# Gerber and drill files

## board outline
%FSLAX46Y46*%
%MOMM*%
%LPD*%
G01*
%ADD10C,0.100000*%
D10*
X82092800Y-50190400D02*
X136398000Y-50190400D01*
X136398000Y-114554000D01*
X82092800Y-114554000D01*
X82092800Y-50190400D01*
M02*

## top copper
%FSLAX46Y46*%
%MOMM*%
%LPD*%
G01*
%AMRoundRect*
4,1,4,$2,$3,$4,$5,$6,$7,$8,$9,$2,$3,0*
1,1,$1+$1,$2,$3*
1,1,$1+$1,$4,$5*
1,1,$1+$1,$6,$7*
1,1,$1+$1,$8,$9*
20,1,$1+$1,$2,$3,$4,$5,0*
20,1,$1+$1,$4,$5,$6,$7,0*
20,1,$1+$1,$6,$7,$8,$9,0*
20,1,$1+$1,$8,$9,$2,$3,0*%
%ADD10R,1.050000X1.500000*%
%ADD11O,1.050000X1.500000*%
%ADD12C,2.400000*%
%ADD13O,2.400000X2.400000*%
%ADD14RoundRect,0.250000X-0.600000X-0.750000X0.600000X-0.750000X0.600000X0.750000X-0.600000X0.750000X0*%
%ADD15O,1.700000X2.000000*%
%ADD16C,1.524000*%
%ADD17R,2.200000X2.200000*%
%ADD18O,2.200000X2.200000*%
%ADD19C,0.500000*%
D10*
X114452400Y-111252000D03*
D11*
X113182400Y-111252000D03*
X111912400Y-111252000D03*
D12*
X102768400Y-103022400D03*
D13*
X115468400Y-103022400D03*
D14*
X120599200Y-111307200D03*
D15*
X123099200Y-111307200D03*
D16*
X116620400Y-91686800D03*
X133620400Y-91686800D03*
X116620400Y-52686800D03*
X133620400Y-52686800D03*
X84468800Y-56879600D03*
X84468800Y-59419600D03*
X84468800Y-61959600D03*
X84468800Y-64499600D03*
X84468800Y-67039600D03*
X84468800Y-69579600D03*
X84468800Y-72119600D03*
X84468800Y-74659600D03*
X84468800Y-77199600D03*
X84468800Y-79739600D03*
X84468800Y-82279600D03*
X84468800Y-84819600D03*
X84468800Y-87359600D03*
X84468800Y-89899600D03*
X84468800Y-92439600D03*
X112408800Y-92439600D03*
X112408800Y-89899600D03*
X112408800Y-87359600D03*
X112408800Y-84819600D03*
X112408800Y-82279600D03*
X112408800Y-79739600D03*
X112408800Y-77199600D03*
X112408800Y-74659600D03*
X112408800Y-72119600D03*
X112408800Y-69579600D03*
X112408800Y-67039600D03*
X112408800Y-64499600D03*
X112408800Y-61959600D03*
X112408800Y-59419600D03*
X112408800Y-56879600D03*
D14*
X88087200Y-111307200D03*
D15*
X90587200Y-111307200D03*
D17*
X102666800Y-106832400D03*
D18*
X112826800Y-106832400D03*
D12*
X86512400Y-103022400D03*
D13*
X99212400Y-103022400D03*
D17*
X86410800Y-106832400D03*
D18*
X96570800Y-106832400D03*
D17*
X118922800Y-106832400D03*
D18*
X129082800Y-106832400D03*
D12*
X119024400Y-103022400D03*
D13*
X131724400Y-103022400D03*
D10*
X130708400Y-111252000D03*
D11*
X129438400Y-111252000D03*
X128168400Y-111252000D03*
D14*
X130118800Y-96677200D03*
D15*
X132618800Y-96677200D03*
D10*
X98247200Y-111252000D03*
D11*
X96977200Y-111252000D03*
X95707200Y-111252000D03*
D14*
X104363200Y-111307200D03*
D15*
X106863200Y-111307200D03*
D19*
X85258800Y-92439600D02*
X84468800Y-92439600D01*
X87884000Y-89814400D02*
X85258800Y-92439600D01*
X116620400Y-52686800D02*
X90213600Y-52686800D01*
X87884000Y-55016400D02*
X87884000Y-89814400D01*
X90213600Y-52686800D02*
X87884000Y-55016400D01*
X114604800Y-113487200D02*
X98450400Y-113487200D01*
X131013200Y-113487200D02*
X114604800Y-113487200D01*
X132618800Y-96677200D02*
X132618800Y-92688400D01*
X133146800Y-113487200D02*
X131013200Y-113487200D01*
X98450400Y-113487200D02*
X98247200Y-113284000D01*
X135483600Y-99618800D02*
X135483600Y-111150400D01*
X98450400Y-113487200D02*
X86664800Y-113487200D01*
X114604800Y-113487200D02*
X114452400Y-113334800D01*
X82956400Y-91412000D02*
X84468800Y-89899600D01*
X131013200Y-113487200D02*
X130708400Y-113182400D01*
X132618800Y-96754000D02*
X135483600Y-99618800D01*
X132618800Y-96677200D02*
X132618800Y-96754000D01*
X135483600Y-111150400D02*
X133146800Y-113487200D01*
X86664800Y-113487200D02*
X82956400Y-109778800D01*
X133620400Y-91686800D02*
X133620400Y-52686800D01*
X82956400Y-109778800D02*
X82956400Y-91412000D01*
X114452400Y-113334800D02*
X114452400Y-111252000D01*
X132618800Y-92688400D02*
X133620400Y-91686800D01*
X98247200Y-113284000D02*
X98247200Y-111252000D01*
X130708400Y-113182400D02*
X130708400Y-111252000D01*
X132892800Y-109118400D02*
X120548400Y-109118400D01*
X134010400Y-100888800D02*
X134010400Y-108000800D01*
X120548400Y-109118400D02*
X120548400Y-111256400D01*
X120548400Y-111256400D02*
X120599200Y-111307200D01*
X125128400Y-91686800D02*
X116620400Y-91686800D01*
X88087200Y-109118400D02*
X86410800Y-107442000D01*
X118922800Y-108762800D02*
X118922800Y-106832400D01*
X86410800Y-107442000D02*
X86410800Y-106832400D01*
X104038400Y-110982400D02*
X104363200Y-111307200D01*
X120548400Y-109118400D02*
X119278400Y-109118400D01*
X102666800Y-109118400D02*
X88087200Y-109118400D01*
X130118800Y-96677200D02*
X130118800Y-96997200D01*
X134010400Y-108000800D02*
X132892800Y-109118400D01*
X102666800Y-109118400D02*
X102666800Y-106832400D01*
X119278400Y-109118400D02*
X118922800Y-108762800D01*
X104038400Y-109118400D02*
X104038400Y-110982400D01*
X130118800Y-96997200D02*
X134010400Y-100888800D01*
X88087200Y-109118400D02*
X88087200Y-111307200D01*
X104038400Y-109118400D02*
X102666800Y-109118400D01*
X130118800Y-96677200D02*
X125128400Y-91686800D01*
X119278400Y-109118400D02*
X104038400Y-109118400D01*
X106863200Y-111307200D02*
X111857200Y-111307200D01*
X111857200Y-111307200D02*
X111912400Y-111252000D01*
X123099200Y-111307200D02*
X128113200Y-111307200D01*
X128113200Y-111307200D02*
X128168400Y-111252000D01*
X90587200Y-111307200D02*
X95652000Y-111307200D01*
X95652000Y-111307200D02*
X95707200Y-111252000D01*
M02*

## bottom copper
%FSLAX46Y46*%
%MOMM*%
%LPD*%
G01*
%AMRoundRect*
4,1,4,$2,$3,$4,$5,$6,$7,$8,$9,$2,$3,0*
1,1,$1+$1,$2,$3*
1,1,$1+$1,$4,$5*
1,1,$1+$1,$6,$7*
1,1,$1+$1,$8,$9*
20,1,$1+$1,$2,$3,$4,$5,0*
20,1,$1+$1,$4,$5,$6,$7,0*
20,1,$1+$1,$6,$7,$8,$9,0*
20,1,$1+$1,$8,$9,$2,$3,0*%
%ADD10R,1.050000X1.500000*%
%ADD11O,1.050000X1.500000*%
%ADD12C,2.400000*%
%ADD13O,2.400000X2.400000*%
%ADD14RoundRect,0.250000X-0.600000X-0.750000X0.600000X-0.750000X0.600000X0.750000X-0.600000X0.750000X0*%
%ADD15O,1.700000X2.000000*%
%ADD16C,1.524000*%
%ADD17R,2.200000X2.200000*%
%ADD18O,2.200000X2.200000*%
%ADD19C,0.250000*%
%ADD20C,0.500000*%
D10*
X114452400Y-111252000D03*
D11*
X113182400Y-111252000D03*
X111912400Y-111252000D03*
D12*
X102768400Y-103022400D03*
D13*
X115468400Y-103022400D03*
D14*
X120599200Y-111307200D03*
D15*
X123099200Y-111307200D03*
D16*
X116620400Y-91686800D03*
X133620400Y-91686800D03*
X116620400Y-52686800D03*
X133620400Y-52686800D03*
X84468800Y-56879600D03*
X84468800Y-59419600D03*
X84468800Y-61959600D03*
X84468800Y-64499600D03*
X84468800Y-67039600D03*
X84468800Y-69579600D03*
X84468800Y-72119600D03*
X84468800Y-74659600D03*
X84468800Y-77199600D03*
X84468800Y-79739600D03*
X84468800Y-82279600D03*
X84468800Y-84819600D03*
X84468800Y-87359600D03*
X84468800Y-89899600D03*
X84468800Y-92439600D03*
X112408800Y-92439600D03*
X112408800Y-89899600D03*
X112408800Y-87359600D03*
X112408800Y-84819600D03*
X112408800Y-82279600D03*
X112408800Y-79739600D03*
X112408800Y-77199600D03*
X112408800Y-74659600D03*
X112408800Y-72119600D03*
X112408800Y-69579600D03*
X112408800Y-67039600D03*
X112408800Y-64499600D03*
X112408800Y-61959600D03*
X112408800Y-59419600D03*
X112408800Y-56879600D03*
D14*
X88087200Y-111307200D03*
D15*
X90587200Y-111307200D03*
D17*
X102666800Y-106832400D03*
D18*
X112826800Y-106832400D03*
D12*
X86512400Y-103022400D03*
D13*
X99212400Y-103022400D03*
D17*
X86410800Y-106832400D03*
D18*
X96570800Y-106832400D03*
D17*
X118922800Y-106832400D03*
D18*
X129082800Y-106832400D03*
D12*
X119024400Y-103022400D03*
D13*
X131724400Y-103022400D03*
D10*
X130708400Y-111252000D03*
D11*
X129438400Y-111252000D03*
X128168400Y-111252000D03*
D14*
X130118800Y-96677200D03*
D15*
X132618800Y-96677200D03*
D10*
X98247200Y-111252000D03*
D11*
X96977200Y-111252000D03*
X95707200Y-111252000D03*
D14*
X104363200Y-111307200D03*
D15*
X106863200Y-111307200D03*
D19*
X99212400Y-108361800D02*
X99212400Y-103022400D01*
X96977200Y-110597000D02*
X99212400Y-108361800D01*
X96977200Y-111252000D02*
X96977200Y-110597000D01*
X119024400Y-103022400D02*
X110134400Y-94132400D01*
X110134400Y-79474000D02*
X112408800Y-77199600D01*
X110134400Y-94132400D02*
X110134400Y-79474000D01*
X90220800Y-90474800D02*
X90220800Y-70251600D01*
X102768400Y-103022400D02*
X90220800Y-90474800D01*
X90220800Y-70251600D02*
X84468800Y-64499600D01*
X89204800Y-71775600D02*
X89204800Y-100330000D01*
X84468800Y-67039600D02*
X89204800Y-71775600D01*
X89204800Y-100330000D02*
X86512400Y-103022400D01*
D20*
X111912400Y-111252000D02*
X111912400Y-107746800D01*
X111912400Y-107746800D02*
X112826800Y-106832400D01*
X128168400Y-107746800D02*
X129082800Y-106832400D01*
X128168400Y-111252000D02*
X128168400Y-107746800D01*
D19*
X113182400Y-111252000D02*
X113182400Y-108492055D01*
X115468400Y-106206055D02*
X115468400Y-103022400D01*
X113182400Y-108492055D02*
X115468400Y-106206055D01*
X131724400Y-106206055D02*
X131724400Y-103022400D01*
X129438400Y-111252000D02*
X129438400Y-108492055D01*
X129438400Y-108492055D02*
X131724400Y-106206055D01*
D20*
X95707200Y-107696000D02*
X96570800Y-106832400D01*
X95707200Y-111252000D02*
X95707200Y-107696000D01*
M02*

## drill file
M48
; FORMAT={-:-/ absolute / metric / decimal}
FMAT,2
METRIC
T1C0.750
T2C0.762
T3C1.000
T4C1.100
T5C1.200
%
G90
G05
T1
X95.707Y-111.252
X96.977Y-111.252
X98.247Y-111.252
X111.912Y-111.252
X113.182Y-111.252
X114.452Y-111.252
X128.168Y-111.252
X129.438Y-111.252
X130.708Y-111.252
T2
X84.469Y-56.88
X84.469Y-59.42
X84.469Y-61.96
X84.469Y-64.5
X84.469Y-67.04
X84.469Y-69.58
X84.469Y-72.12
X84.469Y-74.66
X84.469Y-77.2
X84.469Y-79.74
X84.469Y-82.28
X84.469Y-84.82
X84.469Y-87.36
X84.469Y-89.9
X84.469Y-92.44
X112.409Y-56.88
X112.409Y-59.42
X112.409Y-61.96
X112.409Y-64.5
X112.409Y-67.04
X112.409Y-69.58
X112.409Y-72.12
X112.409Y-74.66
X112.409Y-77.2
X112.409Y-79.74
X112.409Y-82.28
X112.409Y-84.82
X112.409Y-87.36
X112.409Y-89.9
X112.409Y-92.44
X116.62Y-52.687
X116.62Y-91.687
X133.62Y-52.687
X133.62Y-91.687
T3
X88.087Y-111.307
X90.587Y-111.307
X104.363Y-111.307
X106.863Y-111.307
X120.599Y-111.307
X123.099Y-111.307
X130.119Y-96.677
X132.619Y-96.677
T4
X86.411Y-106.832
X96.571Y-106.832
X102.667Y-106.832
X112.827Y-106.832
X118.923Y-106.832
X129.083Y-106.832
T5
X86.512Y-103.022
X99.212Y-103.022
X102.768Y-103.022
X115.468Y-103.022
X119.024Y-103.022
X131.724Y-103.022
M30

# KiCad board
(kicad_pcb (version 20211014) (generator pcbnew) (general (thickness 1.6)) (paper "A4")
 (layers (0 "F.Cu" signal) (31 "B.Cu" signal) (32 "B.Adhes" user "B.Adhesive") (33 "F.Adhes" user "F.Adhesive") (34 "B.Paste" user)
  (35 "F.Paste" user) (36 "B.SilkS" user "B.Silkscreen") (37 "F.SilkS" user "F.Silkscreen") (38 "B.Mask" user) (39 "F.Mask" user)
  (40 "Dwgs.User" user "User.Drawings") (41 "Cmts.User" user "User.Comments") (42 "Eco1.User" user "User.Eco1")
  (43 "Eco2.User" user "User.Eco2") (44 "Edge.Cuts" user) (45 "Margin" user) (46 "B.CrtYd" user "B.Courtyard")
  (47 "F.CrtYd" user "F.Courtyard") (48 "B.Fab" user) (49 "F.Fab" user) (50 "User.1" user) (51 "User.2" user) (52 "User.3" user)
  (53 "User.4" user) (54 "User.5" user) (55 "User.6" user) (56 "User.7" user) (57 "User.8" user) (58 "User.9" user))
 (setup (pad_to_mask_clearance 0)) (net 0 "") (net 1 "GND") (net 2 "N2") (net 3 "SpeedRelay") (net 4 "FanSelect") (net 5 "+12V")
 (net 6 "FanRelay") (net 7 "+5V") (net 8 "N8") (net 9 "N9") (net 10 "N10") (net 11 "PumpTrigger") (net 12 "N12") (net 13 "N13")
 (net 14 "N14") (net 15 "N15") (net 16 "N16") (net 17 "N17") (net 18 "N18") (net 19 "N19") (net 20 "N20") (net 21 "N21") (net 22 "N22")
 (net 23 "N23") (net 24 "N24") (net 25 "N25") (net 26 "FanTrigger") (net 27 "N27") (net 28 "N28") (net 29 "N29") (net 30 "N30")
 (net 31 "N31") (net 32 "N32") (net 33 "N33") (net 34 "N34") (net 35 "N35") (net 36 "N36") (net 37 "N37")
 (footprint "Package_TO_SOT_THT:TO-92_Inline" (layer "F.Cu") (at 114.4524 111.252 180)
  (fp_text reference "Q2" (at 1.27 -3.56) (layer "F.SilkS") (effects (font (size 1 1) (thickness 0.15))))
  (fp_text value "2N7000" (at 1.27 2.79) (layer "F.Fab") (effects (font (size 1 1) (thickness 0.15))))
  (pad "1" thru_hole rect (at 0 0 180) (size 1.05 1.5) (drill 0.75) (layers *.Cu *.Mask) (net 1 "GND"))
  (pad "2" thru_hole oval (at 1.27 0 180) (size 1.05 1.5) (drill 0.75) (layers *.Cu *.Mask) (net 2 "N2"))
  (pad "3" thru_hole oval (at 2.54 0 180) (size 1.05 1.5) (drill 0.75) (layers *.Cu *.Mask) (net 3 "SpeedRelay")))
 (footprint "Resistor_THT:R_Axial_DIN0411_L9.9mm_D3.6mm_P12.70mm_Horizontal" (layer "F.Cu") (at 102.7684 103.0224)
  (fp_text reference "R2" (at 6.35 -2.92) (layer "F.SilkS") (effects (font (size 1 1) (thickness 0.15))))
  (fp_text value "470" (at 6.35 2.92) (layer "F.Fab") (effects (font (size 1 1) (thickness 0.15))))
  (pad "1" thru_hole circle (at 0 0) (size 2.4 2.4) (drill 1.2) (layers *.Cu *.Mask) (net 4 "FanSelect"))
  (pad "2" thru_hole oval (at 12.7 0) (size 2.4 2.4) (drill 1.2) (layers *.Cu *.Mask) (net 2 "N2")))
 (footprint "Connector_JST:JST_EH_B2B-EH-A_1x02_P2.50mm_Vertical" (layer "F.Cu") (at 120.5992 111.3072)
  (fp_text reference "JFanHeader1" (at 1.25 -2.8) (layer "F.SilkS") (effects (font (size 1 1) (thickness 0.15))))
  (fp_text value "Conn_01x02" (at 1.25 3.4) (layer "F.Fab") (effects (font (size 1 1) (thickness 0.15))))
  (pad "1" thru_hole roundrect (at 0 0) (size 1.7 2) (drill 1) (layers *.Cu *.Mask) (roundrect_rratio 0.147059) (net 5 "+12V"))
  (pad "2" thru_hole oval (at 2.5 0) (size 1.7 2) (drill 1) (layers *.Cu *.Mask) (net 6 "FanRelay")))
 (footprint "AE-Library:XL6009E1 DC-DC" (layer "F.Cu") (at 119.7004 83.5268 90)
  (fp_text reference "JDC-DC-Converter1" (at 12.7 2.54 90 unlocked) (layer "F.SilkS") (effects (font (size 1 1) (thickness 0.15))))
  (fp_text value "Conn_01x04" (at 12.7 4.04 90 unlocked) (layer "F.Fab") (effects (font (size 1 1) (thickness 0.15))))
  (pad "1" thru_hole circle (at -8.16 -3.08 90) (size 1.524 1.524) (drill 0.762) (layers *.Cu *.Mask) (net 5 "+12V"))
  (pad "2" thru_hole circle (at -8.16 13.92 90) (size 1.524 1.524) (drill 0.762) (layers *.Cu *.Mask) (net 1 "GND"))
  (pad "3" thru_hole circle (at 30.84 -3.08 90) (size 1.524 1.524) (drill 0.762) (layers *.Cu *.Mask) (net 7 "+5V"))
  (pad "4" thru_hole circle (at 30.84 13.92 90) (size 1.524 1.524) (drill 0.762) (layers *.Cu *.Mask) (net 1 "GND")))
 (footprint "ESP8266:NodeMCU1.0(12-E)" (layer "F.Cu") (at 98.4388 74.6596)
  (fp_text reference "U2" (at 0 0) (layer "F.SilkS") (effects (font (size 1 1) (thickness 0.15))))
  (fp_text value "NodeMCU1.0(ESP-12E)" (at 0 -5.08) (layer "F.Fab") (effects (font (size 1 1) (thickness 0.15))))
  (pad "1" thru_hole circle locked (at -13.97 -17.78) (size 1.524 1.524) (drill 0.762) (layers *.Cu *.Mask "F.SilkS") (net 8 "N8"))
  (pad "2" thru_hole circle locked (at -13.97 -15.24) (size 1.524 1.524) (drill 0.762) (layers *.Cu *.Mask "F.SilkS") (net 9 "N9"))
  (pad "3" thru_hole circle locked (at -13.97 -12.7) (size 1.524 1.524) (drill 0.762) (layers *.Cu *.Mask "F.SilkS") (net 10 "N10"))
  (pad "4" thru_hole circle locked (at -13.97 -10.16) (size 1.524 1.524) (drill 0.762) (layers *.Cu *.Mask "F.SilkS") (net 4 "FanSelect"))
  (pad "5" thru_hole circle locked (at -13.97 -7.62) (size 1.524 1.524) (drill 0.762) (layers *.Cu *.Mask "F.SilkS") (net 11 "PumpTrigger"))
  (pad "6" thru_hole circle locked (at -13.97 -5.08) (size 1.524 1.524) (drill 0.762) (layers *.Cu *.Mask "F.SilkS") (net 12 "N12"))
  (pad "7" thru_hole circle locked (at -13.97 -2.54) (size 1.524 1.524) (drill 0.762) (layers *.Cu *.Mask "F.SilkS") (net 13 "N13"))
  (pad "8" thru_hole circle locked (at -13.97 0) (size 1.524 1.524) (drill 0.762) (layers *.Cu *.Mask "F.SilkS") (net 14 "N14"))
  (pad "9" thru_hole circle locked (at -13.97 2.54) (size 1.524 1.524) (drill 0.762) (layers *.Cu *.Mask "F.SilkS") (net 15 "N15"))
  (pad "10" thru_hole circle locked (at -13.97 5.08) (size 1.524 1.524) (drill 0.762) (layers *.Cu *.Mask "F.SilkS") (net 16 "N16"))
  (pad "11" thru_hole circle locked (at -13.97 7.62) (size 1.524 1.524) (drill 0.762) (layers *.Cu *.Mask "F.SilkS") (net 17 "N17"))
  (pad "12" thru_hole circle locked (at -13.97 10.16) (size 1.524 1.524) (drill 0.762) (layers *.Cu *.Mask "F.SilkS") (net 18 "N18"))
  (pad "13" thru_hole circle locked (at -13.97 12.7) (size 1.524 1.524) (drill 0.762) (layers *.Cu *.Mask "F.SilkS") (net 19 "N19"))
  (pad "14" thru_hole circle locked (at -13.97 15.24) (size 1.524 1.524) (drill 0.762) (layers *.Cu *.Mask "F.SilkS") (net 1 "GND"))
  (pad "15" thru_hole circle locked (at -13.97 17.78) (size 1.524 1.524) (drill 0.762) (layers *.Cu *.Mask "F.SilkS") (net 7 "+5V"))
  (pad "16" thru_hole circle locked (at 13.97 17.78) (size 1.524 1.524) (drill 0.762) (layers *.Cu *.Mask "F.SilkS") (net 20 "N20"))
  (pad "17" thru_hole circle locked (at 13.97 15.24) (size 1.524 1.524) (drill 0.762) (layers *.Cu *.Mask "F.SilkS") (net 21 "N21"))
  (pad "18" thru_hole circle locked (at 13.97 12.7) (size 1.524 1.524) (drill 0.762) (layers *.Cu *.Mask "F.SilkS") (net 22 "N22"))
  (pad "19" thru_hole circle locked (at 13.97 10.16) (size 1.524 1.524) (drill 0.762) (layers *.Cu *.Mask "F.SilkS") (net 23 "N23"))
  (pad "20" thru_hole circle locked (at 13.97 7.62) (size 1.524 1.524) (drill 0.762) (layers *.Cu *.Mask "F.SilkS") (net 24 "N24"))
  (pad "21" thru_hole circle locked (at 13.97 5.08) (size 1.524 1.524) (drill 0.762) (layers *.Cu *.Mask "F.SilkS") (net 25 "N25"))
  (pad "22" thru_hole circle locked (at 13.97 2.54) (size 1.524 1.524) (drill 0.762) (layers *.Cu *.Mask "F.SilkS") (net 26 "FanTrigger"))
  (pad "23" thru_hole circle locked (at 13.97 0) (size 1.524 1.524) (drill 0.762) (layers *.Cu *.Mask "F.SilkS") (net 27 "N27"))
  (pad "24" thru_hole circle locked (at 13.97 -2.54) (size 1.524 1.524) (drill 0.762) (layers *.Cu *.Mask "F.SilkS") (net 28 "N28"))
  (pad "25" thru_hole circle locked (at 13.97 -5.08) (size 1.524 1.524) (drill 0.762) (layers *.Cu *.Mask "F.SilkS") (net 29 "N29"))
  (pad "26" thru_hole circle locked (at 13.97 -7.62) (size 1.524 1.524) (drill 0.762) (layers *.Cu *.Mask "F.SilkS") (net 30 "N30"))
  (pad "27" thru_hole circle locked (at 13.97 -10.16) (size 1.524 1.524) (drill 0.762) (layers *.Cu *.Mask "F.SilkS") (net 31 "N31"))
  (pad "28" thru_hole circle locked (at 13.97 -12.7) (size 1.524 1.524) (drill 0.762) (layers *.Cu *.Mask "F.SilkS") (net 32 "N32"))
  (pad "29" thru_hole circle locked (at 13.97 -15.24) (size 1.524 1.524) (drill 0.762) (layers *.Cu *.Mask "F.SilkS") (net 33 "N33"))
  (pad "30" thru_hole circle locked (at 13.97 -17.78) (size 1.524 1.524) (drill 0.762) (layers *.Cu *.Mask "F.SilkS") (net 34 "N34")))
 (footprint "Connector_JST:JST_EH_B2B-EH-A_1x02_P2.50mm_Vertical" (layer "F.Cu") (at 88.0872 111.3072)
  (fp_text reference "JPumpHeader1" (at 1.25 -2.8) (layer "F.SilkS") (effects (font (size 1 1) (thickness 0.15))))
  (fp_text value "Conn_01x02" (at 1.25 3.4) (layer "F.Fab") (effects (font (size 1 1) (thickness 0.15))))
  (pad "1" thru_hole roundrect (at 0 0) (size 1.7 2) (drill 1) (layers *.Cu *.Mask) (roundrect_rratio 0.147059) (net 5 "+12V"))
  (pad "2" thru_hole oval (at 2.5 0) (size 1.7 2) (drill 1) (layers *.Cu *.Mask) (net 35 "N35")))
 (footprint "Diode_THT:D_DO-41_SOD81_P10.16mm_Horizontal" (layer "F.Cu") (at 102.6668 106.8324)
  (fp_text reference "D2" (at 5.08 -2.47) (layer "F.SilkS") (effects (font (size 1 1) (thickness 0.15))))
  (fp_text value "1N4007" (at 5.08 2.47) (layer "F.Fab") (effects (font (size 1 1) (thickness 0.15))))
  (pad "1" thru_hole rect (at 0 0) (size 2.2 2.2) (drill 1.1) (layers *.Cu *.Mask) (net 5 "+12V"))
  (pad "2" thru_hole oval (at 10.16 0) (size 2.2 2.2) (drill 1.1) (layers *.Cu *.Mask) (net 3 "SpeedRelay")))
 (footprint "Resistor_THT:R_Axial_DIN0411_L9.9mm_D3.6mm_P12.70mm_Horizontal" (layer "F.Cu") (at 86.5124 103.0224)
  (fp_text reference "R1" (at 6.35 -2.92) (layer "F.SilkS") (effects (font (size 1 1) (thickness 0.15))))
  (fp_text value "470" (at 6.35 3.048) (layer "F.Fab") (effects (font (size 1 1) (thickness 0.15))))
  (pad "1" thru_hole circle (at 0 0) (size 2.4 2.4) (drill 1.2) (layers *.Cu *.Mask) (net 11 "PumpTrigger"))
  (pad "2" thru_hole oval (at 12.7 0) (size 2.4 2.4) (drill 1.2) (layers *.Cu *.Mask) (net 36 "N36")))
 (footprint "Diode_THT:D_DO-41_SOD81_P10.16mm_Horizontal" (layer "F.Cu") (at 86.4108 106.8324)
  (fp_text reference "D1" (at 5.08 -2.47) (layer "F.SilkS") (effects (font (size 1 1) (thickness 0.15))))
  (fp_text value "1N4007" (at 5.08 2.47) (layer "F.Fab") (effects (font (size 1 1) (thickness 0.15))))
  (pad "1" thru_hole rect (at 0 0) (size 2.2 2.2) (drill 1.1) (layers *.Cu *.Mask) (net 5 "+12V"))
  (pad "2" thru_hole oval (at 10.16 0) (size 2.2 2.2) (drill 1.1) (layers *.Cu *.Mask) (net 35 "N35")))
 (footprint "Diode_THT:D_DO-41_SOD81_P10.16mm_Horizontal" (layer "F.Cu") (at 118.9228 106.8324)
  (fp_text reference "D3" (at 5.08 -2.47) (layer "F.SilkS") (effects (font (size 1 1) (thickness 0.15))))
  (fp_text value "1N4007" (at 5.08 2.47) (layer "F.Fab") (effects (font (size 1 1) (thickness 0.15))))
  (pad "1" thru_hole rect (at 0 0) (size 2.2 2.2) (drill 1.1) (layers *.Cu *.Mask) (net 5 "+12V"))
  (pad "2" thru_hole oval (at 10.16 0) (size 2.2 2.2) (drill 1.1) (layers *.Cu *.Mask) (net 6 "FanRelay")))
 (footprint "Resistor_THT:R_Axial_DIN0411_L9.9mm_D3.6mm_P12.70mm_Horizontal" (layer "F.Cu") (at 119.0244 103.0224)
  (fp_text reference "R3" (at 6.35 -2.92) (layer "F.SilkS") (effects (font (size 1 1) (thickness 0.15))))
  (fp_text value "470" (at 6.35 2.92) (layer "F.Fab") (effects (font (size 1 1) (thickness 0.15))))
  (pad "1" thru_hole circle (at 0 0) (size 2.4 2.4) (drill 1.2) (layers *.Cu *.Mask) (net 26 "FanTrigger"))
  (pad "2" thru_hole oval (at 12.7 0) (size 2.4 2.4) (drill 1.2) (layers *.Cu *.Mask) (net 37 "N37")))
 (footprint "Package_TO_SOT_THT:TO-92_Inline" (layer "F.Cu") (at 130.7084 111.252 180)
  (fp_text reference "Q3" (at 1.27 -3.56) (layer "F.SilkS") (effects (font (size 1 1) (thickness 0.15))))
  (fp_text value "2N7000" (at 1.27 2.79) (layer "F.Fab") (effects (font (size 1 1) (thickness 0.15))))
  (pad "1" thru_hole rect (at 0 0 180) (size 1.05 1.5) (drill 0.75) (layers *.Cu *.Mask) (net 1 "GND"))
  (pad "2" thru_hole oval (at 1.27 0 180) (size 1.05 1.5) (drill 0.75) (layers *.Cu *.Mask) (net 37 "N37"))
  (pad "3" thru_hole oval (at 2.54 0 180) (size 1.05 1.5) (drill 0.75) (layers *.Cu *.Mask) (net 6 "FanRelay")))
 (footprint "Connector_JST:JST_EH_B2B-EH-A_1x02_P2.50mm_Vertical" (layer "F.Cu") (at 130.1188 96.6772)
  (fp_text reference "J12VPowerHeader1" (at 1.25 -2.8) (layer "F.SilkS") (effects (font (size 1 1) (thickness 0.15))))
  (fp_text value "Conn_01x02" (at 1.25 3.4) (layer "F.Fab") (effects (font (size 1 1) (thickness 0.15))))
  (pad "1" thru_hole roundrect (at 0 0) (size 1.7 2) (drill 1) (layers *.Cu *.Mask) (roundrect_rratio 0.147059) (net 5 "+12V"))
  (pad "2" thru_hole oval (at 2.5 0) (size 1.7 2) (drill 1) (layers *.Cu *.Mask) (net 1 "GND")))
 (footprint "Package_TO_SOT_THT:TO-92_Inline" (layer "F.Cu") (at 98.2472 111.252 180)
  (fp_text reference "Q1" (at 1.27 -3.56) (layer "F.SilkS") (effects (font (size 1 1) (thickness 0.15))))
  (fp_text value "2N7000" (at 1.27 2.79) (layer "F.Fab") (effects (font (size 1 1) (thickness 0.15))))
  (pad "1" thru_hole rect (at 0 0 180) (size 1.05 1.5) (drill 0.75) (layers *.Cu *.Mask) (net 1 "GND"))
  (pad "2" thru_hole oval (at 1.27 0 180) (size 1.05 1.5) (drill 0.75) (layers *.Cu *.Mask) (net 36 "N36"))
  (pad "3" thru_hole oval (at 2.54 0 180) (size 1.05 1.5) (drill 0.75) (layers *.Cu *.Mask) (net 35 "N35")))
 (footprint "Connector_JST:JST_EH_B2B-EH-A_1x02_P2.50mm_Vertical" (layer "F.Cu") (at 104.3632 111.3072)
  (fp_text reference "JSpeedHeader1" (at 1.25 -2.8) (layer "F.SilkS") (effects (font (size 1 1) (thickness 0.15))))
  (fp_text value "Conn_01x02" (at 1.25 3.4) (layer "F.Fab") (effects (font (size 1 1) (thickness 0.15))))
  (pad "1" thru_hole roundrect (at 0 0) (size 1.7 2) (drill 1) (layers *.Cu *.Mask) (roundrect_rratio 0.147059) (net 5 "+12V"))
  (pad "2" thru_hole oval (at 2.5 0) (size 1.7 2) (drill 1) (layers *.Cu *.Mask) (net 3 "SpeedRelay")))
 (gr_rect (start 82.0928 114.554) (end 136.398 50.1904) (layer "Edge.Cuts") (width 0.1) (fill none))
 (segment (start 85.2588 92.4396) (end 84.4688 92.4396) (width 0.5) (layer "F.Cu") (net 7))
 (segment (start 87.884 89.8144) (end 85.2588 92.4396) (width 0.5) (layer "F.Cu") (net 7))
 (segment (start 116.6204 52.6868) (end 90.2136 52.6868) (width 0.5) (layer "F.Cu") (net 7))
 (segment (start 87.884 55.0164) (end 87.884 89.8144) (width 0.5) (layer "F.Cu") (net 7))
 (segment (start 90.2136 52.6868) (end 87.884 55.0164) (width 0.5) (layer "F.Cu") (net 7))
 (segment (start 114.6048 113.4872) (end 98.4504 113.4872) (width 0.5) (layer "F.Cu") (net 1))
 (segment (start 131.0132 113.4872) (end 114.6048 113.4872) (width 0.5) (layer "F.Cu") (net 1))
 (segment (start 132.6188 96.6772) (end 132.6188 92.6884) (width 0.5) (layer "F.Cu") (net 1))
 (segment (start 133.1468 113.4872) (end 131.0132 113.4872) (width 0.5) (layer "F.Cu") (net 1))
 (segment (start 98.4504 113.4872) (end 98.2472 113.284) (width 0.5) (layer "F.Cu") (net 1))
 (segment (start 135.4836 99.6188) (end 135.4836 111.1504) (width 0.5) (layer "F.Cu") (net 1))
 (segment (start 98.4504 113.4872) (end 86.6648 113.4872) (width 0.5) (layer "F.Cu") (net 1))
 (segment (start 114.6048 113.4872) (end 114.4524 113.3348) (width 0.5) (layer "F.Cu") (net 1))
 (segment (start 82.9564 91.412) (end 84.4688 89.8996) (width 0.5) (layer "F.Cu") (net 1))
 (segment (start 131.0132 113.4872) (end 130.7084 113.1824) (width 0.5) (layer "F.Cu") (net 1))
 (segment (start 132.6188 96.754) (end 135.4836 99.6188) (width 0.5) (layer "F.Cu") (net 1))
 (segment (start 132.6188 96.6772) (end 132.6188 96.754) (width 0.5) (layer "F.Cu") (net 1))
 (segment (start 135.4836 111.1504) (end 133.1468 113.4872) (width 0.5) (layer "F.Cu") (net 1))
 (segment (start 86.6648 113.4872) (end 82.9564 109.7788) (width 0.5) (layer "F.Cu") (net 1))
 (segment (start 133.6204 91.6868) (end 133.6204 52.6868) (width 0.5) (layer "F.Cu") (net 1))
 (segment (start 82.9564 109.7788) (end 82.9564 91.412) (width 0.5) (layer "F.Cu") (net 1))
 (segment (start 114.4524 113.3348) (end 114.4524 111.252) (width 0.5) (layer "F.Cu") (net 1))
 (segment (start 132.6188 92.6884) (end 133.6204 91.6868) (width 0.5) (layer "F.Cu") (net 1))
 (segment (start 98.2472 113.284) (end 98.2472 111.252) (width 0.5) (layer "F.Cu") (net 1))
 (segment (start 130.7084 113.1824) (end 130.7084 111.252) (width 0.5) (layer "F.Cu") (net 1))
 (segment (start 99.2124 108.3618) (end 99.2124 103.0224) (width 0.25) (layer "B.Cu") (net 36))
 (segment (start 96.9772 110.597) (end 99.2124 108.3618) (width 0.25) (layer "B.Cu") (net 36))
 (segment (start 96.9772 111.252) (end 96.9772 110.597) (width 0.25) (layer "B.Cu") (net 36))
 (segment (start 119.0244 103.0224) (end 110.1344 94.1324) (width 0.25) (layer "B.Cu") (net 26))
 (segment (start 110.1344 79.474) (end 112.4088 77.1996) (width 0.25) (layer "B.Cu") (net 26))
 (segment (start 110.1344 94.1324) (end 110.1344 79.474) (width 0.25) (layer "B.Cu") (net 26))
 (segment (start 90.2208 90.4748) (end 90.2208 70.2516) (width 0.25) (layer "B.Cu") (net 4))
 (segment (start 102.7684 103.0224) (end 90.2208 90.4748) (width 0.25) (layer "B.Cu") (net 4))
 (segment (start 90.2208 70.2516) (end 84.4688 64.4996) (width 0.25) (layer "B.Cu") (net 4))
 (segment (start 89.2048 71.7756) (end 89.2048 100.33) (width 0.25) (layer "B.Cu") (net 11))
 (segment (start 84.4688 67.0396) (end 89.2048 71.7756) (width 0.25) (layer "B.Cu") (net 11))
 (segment (start 89.2048 100.33) (end 86.5124 103.0224) (width 0.25) (layer "B.Cu") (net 11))
 (segment (start 132.8928 109.1184) (end 120.5484 109.1184) (width 0.5) (layer "F.Cu") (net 5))
 (segment (start 134.0104 100.8888) (end 134.0104 108.0008) (width 0.5) (layer "F.Cu") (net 5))
 (segment (start 120.5484 109.1184) (end 120.5484 111.2564) (width 0.5) (layer "F.Cu") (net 5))
 (segment (start 120.5484 111.2564) (end 120.5992 111.3072) (width 0.5) (layer "F.Cu") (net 5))
 (segment (start 125.1284 91.6868) (end 116.6204 91.6868) (width 0.5) (layer "F.Cu") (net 5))
 (segment (start 88.0872 109.1184) (end 86.4108 107.442) (width 0.5) (layer "F.Cu") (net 5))
 (segment (start 118.9228 108.7628) (end 118.9228 106.8324) (width 0.5) (layer "F.Cu") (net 5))
 (segment (start 86.4108 107.442) (end 86.4108 106.8324) (width 0.5) (layer "F.Cu") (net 5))
 (segment (start 104.0384 110.9824) (end 104.3632 111.3072) (width 0.5) (layer "F.Cu") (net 5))
 (segment (start 120.5484 109.1184) (end 119.2784 109.1184) (width 0.5) (layer "F.Cu") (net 5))
 (segment (start 102.6668 109.1184) (end 88.0872 109.1184) (width 0.5) (layer "F.Cu") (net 5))
 (segment (start 130.1188 96.6772) (end 130.1188 96.9972) (width 0.5) (layer "F.Cu") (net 5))
 (segment (start 134.0104 108.0008) (end 132.8928 109.1184) (width 0.5) (layer "F.Cu") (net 5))
 (segment (start 102.6668 109.1184) (end 102.6668 106.8324) (width 0.5) (layer "F.Cu") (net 5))
 (segment (start 119.2784 109.1184) (end 118.9228 108.7628) (width 0.5) (layer "F.Cu") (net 5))
 (segment (start 104.0384 109.1184) (end 104.0384 110.9824) (width 0.5) (layer "F.Cu") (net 5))
 (segment (start 130.1188 96.9972) (end 134.0104 100.8888) (width 0.5) (layer "F.Cu") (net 5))
 (segment (start 88.0872 109.1184) (end 88.0872 111.3072) (width 0.5) (layer "F.Cu") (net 5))
 (segment (start 104.0384 109.1184) (end 102.6668 109.1184) (width 0.5) (layer "F.Cu") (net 5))
 (segment (start 130.1188 96.6772) (end 125.1284 91.6868) (width 0.5) (layer "F.Cu") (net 5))
 (segment (start 119.2784 109.1184) (end 104.0384 109.1184) (width 0.5) (layer "F.Cu") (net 5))
 (segment (start 106.8632 111.3072) (end 111.8572 111.3072) (width 0.5) (layer "F.Cu") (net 3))
 (segment (start 111.8572 111.3072) (end 111.9124 111.252) (width 0.5) (layer "F.Cu") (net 3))
 (segment (start 111.9124 111.252) (end 111.9124 107.7468) (width 0.5) (layer "B.Cu") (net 3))
 (segment (start 111.9124 107.7468) (end 112.8268 106.8324) (width 0.5) (layer "B.Cu") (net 3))
 (segment (start 123.0992 111.3072) (end 128.1132 111.3072) (width 0.5) (layer "F.Cu") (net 6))
 (segment (start 128.1132 111.3072) (end 128.1684 111.252) (width 0.5) (layer "F.Cu") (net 6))
 (segment (start 128.1684 107.7468) (end 129.0828 106.8324) (width 0.5) (layer "B.Cu") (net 6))
 (segment (start 128.1684 111.252) (end 128.1684 107.7468) (width 0.5) (layer "B.Cu") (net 6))
 (segment (start 113.1824 111.252) (end 113.1824 108.492055) (width 0.25) (layer "B.Cu") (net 2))
 (segment (start 115.4684 106.206055) (end 115.4684 103.0224) (width 0.25) (layer "B.Cu") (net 2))
 (segment (start 113.1824 108.492055) (end 115.4684 106.206055) (width 0.25) (layer "B.Cu") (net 2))
 (segment (start 131.7244 106.206055) (end 131.7244 103.0224) (width 0.25) (layer "B.Cu") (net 37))
 (segment (start 129.4384 111.252) (end 129.4384 108.492055) (width 0.25) (layer "B.Cu") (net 37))
 (segment (start 129.4384 108.492055) (end 131.7244 106.206055) (width 0.25) (layer "B.Cu") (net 37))
 (segment (start 90.5872 111.3072) (end 95.652 111.3072) (width 0.5) (layer "F.Cu") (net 35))
 (segment (start 95.652 111.3072) (end 95.7072 111.252) (width 0.5) (layer "F.Cu") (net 35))
 (segment (start 95.7072 107.696) (end 96.5708 106.8324) (width 0.5) (layer "B.Cu") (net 35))
 (segment (start 95.7072 111.252) (end 95.7072 107.696) (width 0.5) (layer "B.Cu") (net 35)))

